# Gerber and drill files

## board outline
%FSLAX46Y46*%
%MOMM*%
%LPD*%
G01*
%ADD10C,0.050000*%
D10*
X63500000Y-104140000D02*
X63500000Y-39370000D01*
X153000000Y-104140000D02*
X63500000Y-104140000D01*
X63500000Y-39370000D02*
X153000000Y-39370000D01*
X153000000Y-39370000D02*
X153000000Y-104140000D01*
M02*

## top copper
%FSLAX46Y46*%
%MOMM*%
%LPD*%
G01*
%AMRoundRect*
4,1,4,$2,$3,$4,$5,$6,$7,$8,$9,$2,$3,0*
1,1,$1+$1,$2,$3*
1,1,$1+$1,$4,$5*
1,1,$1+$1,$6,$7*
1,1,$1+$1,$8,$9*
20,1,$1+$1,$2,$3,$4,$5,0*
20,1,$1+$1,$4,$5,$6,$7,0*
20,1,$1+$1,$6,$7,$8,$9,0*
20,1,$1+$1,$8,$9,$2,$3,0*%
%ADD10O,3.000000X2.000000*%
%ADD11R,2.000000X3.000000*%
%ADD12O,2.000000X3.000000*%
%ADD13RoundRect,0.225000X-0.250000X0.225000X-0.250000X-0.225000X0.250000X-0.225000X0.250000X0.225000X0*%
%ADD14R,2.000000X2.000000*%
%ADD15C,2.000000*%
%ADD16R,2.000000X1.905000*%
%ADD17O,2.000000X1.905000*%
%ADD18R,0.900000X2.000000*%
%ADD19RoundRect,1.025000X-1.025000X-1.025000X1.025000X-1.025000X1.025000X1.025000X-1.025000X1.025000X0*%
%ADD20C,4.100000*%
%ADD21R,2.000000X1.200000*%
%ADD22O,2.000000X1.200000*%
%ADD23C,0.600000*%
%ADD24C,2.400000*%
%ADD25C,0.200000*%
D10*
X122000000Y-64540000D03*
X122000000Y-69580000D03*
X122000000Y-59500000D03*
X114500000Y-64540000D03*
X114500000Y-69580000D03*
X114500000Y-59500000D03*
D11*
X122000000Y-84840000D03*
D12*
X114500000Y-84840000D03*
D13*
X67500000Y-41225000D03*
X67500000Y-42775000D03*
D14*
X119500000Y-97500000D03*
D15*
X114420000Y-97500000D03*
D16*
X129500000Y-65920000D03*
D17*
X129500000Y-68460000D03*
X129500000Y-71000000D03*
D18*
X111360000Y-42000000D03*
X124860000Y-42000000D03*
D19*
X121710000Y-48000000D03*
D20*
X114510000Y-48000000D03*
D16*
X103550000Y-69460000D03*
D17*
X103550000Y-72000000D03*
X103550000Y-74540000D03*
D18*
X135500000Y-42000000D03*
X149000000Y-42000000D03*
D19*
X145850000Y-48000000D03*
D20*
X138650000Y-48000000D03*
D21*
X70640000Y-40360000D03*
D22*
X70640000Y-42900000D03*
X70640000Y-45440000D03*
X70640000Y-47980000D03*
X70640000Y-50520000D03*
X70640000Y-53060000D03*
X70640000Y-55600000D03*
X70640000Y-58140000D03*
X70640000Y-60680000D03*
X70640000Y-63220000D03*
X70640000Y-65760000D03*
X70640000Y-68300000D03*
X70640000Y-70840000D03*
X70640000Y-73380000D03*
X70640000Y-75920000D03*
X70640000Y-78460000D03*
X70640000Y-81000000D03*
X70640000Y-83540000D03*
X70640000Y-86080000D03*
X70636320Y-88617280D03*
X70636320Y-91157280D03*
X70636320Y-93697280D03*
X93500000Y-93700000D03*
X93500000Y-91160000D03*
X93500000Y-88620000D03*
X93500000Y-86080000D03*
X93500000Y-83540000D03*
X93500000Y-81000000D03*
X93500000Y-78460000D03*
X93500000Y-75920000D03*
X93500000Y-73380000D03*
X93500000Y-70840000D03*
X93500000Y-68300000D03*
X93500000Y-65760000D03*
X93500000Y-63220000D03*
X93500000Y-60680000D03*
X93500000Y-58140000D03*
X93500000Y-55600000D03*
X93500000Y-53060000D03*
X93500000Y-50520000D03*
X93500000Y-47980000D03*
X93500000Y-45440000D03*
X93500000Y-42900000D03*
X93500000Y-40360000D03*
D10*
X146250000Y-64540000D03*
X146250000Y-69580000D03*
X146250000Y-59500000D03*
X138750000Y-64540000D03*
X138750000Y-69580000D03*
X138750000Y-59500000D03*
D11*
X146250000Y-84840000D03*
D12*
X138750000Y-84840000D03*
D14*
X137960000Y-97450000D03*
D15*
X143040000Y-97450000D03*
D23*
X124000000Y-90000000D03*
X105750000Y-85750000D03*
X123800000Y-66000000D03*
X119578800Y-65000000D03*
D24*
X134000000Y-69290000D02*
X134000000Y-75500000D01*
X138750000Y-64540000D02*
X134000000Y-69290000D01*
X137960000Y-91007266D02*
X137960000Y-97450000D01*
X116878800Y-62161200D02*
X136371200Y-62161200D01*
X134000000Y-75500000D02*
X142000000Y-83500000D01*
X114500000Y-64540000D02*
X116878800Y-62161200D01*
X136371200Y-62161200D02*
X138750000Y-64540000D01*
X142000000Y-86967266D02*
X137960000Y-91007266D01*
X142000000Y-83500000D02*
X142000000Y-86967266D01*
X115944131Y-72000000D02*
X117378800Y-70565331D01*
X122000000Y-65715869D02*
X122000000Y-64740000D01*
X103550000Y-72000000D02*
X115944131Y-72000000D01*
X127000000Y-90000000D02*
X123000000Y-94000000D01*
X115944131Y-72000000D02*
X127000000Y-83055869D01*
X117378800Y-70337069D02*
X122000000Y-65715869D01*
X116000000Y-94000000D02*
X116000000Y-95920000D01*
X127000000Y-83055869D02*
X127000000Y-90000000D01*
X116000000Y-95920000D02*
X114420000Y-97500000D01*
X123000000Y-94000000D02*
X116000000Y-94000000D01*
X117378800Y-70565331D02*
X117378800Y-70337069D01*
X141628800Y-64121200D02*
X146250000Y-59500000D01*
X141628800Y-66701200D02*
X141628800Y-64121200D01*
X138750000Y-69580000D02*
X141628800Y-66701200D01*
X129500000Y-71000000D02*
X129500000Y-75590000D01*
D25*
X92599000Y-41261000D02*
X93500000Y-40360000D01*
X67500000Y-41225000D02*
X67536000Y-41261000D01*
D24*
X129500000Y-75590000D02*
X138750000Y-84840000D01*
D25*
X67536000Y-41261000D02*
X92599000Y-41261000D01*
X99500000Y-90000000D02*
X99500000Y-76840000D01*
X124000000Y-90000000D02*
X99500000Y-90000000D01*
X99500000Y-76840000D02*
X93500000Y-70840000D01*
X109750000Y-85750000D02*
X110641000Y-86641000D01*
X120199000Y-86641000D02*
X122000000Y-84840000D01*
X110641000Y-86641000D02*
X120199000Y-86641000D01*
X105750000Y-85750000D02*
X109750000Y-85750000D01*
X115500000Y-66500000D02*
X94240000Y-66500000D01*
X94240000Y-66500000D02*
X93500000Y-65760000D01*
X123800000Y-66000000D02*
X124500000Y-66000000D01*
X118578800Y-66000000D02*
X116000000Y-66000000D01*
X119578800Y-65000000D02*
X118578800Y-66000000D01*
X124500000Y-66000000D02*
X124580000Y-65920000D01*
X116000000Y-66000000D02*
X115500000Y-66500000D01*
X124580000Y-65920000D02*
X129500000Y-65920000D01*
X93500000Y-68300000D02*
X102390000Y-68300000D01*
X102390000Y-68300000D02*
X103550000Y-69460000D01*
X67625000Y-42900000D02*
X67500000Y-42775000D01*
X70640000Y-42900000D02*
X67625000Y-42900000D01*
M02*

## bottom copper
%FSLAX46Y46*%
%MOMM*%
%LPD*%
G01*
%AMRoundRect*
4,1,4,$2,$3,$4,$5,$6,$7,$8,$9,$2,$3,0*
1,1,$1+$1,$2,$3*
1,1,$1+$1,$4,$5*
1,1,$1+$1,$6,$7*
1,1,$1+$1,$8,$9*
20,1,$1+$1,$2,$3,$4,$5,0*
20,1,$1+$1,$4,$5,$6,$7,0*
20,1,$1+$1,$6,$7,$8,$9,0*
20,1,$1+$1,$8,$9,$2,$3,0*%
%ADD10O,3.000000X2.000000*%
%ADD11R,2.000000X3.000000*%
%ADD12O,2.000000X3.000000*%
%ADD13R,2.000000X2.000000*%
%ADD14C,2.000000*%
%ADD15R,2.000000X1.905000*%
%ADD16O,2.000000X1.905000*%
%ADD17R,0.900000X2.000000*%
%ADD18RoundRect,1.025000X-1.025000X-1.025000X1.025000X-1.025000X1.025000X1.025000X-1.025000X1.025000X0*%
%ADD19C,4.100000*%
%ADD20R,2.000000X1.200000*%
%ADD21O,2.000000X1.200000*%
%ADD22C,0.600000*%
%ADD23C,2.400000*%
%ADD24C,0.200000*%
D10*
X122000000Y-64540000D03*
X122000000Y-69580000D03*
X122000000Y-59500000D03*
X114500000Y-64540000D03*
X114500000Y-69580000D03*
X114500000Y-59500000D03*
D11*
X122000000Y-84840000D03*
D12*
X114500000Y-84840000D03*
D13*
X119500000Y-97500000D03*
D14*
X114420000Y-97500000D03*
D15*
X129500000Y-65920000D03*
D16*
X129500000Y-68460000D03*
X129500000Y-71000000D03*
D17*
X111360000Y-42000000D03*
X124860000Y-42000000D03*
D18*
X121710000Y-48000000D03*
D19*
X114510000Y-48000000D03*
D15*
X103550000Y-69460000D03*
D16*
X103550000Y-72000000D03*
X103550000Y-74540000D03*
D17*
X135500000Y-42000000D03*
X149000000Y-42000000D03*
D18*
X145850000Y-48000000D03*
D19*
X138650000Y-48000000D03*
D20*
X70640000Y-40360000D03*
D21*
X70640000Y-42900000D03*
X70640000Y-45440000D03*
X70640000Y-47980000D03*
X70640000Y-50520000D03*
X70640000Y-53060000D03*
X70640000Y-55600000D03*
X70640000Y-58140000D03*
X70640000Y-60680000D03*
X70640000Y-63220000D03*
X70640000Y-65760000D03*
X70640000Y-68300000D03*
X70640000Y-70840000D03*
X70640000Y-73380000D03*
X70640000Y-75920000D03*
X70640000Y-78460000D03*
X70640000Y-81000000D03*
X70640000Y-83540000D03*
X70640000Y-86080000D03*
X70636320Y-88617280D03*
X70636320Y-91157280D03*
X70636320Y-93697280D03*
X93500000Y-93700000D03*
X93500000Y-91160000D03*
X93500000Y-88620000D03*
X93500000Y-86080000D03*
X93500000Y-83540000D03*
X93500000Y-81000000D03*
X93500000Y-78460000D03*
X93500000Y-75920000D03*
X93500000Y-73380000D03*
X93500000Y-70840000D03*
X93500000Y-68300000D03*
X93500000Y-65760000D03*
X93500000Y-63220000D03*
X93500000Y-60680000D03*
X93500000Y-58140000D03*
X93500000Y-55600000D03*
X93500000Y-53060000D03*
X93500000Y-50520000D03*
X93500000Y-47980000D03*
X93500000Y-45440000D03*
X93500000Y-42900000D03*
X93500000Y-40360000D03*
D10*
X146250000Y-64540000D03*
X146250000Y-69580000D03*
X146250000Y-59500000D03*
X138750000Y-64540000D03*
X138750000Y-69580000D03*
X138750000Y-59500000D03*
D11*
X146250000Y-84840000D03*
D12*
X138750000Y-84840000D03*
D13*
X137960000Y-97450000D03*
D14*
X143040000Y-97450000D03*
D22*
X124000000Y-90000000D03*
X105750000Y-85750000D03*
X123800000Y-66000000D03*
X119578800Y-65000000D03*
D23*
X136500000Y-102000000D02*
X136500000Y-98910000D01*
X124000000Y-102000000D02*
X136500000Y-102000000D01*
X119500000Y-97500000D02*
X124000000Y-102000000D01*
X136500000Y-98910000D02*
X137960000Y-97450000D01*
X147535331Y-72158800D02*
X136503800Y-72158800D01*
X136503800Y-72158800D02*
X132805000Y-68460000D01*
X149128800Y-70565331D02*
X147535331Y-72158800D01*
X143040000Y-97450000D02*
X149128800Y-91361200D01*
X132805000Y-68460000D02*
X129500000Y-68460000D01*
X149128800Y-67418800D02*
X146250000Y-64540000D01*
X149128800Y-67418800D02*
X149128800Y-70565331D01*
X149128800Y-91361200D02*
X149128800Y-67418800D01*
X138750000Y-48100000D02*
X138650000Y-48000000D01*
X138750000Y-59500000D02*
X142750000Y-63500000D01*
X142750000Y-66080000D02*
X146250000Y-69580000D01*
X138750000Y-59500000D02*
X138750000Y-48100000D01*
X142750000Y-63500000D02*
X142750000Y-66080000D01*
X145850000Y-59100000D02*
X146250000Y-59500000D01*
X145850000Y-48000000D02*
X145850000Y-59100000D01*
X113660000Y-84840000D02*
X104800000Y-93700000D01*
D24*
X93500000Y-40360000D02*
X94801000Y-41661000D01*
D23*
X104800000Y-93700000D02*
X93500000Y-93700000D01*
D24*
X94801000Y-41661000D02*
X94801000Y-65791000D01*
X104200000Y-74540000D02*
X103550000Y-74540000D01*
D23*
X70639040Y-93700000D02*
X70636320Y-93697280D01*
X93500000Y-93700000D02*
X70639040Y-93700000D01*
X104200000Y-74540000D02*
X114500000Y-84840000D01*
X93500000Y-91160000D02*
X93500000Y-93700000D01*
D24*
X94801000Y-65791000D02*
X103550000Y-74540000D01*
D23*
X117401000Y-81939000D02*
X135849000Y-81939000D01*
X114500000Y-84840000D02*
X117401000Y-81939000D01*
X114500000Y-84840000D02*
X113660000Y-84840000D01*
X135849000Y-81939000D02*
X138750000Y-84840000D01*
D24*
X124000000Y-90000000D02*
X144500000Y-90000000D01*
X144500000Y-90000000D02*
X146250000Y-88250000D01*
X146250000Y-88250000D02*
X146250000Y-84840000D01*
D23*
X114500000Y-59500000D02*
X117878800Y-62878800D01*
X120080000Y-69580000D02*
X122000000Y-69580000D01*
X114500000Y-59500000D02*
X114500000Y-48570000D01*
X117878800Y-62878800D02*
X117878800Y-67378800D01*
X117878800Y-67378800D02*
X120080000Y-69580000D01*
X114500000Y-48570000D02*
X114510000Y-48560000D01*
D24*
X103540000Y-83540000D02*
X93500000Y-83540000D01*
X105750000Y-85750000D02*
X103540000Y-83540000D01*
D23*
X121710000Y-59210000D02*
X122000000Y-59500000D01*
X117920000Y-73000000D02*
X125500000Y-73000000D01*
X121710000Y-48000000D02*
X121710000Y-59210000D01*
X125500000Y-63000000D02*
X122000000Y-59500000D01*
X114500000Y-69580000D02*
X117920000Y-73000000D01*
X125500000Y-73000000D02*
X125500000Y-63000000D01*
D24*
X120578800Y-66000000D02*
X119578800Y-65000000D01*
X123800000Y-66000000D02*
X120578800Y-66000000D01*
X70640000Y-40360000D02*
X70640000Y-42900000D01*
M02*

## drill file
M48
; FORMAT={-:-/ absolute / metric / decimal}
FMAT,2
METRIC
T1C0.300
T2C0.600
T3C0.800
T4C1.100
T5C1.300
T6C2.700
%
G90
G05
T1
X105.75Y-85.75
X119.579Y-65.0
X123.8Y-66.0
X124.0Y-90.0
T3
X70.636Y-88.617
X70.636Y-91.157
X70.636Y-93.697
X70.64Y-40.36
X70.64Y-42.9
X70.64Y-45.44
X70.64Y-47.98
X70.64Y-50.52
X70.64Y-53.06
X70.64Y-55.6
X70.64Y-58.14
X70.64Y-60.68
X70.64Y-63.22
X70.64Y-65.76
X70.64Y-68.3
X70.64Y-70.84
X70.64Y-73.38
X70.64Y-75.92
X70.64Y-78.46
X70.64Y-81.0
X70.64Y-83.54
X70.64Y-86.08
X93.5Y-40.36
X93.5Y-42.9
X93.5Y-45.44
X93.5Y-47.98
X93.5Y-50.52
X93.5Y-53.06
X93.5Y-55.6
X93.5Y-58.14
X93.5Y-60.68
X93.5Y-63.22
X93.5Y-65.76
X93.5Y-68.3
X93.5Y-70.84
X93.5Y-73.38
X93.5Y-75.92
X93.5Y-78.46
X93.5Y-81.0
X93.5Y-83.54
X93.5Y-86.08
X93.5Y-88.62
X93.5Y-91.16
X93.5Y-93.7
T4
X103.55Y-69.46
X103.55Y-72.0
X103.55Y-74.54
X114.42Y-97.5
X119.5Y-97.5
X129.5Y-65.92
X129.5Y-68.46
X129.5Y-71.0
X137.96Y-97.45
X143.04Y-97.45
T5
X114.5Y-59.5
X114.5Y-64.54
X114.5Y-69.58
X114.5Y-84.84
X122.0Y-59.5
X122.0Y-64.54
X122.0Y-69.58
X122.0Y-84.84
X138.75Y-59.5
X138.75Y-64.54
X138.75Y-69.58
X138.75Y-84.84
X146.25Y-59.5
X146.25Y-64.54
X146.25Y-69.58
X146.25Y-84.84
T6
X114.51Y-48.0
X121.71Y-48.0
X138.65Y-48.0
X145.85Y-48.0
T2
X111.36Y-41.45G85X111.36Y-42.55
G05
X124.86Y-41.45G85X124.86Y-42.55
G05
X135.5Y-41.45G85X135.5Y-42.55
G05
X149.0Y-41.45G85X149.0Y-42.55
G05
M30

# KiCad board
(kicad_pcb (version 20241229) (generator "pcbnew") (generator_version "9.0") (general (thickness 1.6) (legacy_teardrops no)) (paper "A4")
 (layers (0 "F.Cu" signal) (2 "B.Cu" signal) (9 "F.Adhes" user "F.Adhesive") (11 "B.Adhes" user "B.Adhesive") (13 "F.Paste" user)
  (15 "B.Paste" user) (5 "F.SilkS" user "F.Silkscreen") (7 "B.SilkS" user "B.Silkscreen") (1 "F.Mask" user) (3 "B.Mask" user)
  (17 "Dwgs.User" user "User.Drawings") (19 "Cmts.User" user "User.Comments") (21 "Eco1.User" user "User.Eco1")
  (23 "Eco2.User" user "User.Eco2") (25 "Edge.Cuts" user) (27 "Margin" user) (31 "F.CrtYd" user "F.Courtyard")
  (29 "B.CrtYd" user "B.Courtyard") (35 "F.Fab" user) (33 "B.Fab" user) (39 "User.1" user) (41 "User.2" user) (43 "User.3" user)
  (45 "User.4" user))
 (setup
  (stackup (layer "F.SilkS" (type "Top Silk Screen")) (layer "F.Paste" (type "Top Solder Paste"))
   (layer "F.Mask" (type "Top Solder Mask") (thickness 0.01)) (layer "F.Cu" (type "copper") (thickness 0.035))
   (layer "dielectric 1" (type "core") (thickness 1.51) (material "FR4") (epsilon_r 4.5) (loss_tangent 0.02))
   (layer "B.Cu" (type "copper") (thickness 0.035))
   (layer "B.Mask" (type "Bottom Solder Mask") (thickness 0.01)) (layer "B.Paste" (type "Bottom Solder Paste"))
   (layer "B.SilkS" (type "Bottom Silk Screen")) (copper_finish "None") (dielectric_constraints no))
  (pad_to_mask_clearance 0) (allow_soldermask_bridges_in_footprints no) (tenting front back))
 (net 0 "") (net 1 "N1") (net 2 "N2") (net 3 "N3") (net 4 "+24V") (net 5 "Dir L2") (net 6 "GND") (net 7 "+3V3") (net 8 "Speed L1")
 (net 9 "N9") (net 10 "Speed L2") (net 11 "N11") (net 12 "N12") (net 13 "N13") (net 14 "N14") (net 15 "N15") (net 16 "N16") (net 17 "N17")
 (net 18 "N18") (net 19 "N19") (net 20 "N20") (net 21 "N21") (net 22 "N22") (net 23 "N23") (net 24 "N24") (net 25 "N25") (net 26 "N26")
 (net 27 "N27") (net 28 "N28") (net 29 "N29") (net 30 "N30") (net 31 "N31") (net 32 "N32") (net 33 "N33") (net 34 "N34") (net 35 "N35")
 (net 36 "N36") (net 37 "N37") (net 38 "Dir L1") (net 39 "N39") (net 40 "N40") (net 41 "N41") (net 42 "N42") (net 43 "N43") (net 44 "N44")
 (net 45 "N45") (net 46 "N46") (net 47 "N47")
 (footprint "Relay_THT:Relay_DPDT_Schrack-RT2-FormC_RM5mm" (layer "F.Cu") (at 122 84.84 90)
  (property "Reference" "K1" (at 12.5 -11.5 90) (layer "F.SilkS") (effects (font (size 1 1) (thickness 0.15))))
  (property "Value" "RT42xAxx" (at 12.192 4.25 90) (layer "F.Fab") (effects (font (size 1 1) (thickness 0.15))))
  (pad "11" thru_hole oval (at 20.3 0 270) (size 2 3) (drill 1.3) (layers "*.Cu" "*.Mask") (remove_unused_layers no) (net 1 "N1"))
  (pad "12" thru_hole oval (at 15.26 0 270) (size 2 3) (drill 1.3) (layers "*.Cu" "*.Mask") (remove_unused_layers no) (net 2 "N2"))
  (pad "14" thru_hole oval (at 25.34 0 270) (size 2 3) (drill 1.3) (layers "*.Cu" "*.Mask") (remove_unused_layers no) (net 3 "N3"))
  (pad "21" thru_hole oval (at 20.3 -7.5 270) (size 2 3) (drill 1.3) (layers "*.Cu" "*.Mask") (remove_unused_layers no) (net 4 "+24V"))
  (pad "22" thru_hole oval (at 15.26 -7.5 270) (size 2 3) (drill 1.3) (layers "*.Cu" "*.Mask") (remove_unused_layers no) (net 3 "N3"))
  (pad "24" thru_hole oval (at 25.34 -7.5 270) (size 2 3) (drill 1.3) (layers "*.Cu" "*.Mask") (remove_unused_layers no) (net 2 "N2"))
  (pad "A1" thru_hole rect (at 0 0 270) (size 3 2) (drill 1.3) (layers "*.Cu" "*.Mask") (remove_unused_layers no) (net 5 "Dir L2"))
  (pad "A2" thru_hole oval (at 0 -7.5 270) (size 3 2) (drill 1.3) (layers "*.Cu" "*.Mask") (remove_unused_layers no) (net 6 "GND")))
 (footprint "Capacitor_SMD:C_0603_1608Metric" (layer "F.Cu") (at 67.5 42 -90)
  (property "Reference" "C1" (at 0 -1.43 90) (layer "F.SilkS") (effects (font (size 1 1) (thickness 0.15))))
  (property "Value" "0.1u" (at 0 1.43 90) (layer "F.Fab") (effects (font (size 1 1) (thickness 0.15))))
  (pad "1" smd roundrect (at -0.775 0 270) (size 0.9 0.95) (layers "F.Cu" "F.Mask" "F.Paste") (roundrect_rratio 0.25) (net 6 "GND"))
  (pad "2" smd roundrect (at 0.775 0 270) (size 0.9 0.95) (layers "F.Cu" "F.Mask" "F.Paste") (roundrect_rratio 0.25) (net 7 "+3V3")))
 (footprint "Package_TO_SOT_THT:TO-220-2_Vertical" (layer "F.Cu") (at 119.5 97.5 180)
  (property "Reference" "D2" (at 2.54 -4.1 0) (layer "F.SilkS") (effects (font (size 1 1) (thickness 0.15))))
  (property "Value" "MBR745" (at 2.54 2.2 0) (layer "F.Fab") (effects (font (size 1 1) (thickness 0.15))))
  (pad "1" thru_hole rect (at 0 0 180) (size 2 2) (drill 1.1) (layers "*.Cu" "*.Mask") (remove_unused_layers no) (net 4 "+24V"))
  (pad "2" thru_hole circle (at 5.08 0 180) (size 2 2) (drill 1.1) (layers "*.Cu" "*.Mask") (remove_unused_layers no) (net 1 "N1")))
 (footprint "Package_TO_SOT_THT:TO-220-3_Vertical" (layer "F.Cu") (at 129.5 65.92 -90)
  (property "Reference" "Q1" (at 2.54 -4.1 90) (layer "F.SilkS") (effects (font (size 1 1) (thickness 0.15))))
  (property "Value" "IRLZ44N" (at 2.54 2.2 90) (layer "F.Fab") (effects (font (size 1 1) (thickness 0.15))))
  (pad "1" thru_hole rect (at 0 0 270) (size 1.905 2) (drill 1.1) (layers "*.Cu" "*.Mask") (remove_unused_layers no) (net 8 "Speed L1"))
  (pad "2" thru_hole oval (at 2.54 0 270) (size 1.905 2) (drill 1.1) (layers "*.Cu" "*.Mask") (remove_unused_layers no) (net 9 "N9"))
  (pad "3" thru_hole oval (at 5.08 0 270) (size 1.905 2) (drill 1.1) (layers "*.Cu" "*.Mask") (remove_unused_layers no) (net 6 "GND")))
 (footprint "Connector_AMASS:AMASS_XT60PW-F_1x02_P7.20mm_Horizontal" (layer "F.Cu") (at 121.71 48)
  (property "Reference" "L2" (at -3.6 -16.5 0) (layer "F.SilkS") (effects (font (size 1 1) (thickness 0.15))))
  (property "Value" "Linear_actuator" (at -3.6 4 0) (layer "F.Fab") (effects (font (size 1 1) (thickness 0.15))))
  (pad "" thru_hole rect (at -10.35 -6) (size 0.9 2) (drill oval 0.6 1.7) (layers "*.Cu" "*.Mask") (remove_unused_layers no))
  (pad "" thru_hole rect (at 3.15 -6) (size 0.9 2) (drill oval 0.6 1.7) (layers "*.Cu" "*.Mask") (remove_unused_layers no))
  (pad "1" thru_hole roundrect (at 0 0) (size 4.1 4.1) (drill 2.7) (layers "*.Cu" "*.Mask") (remove_unused_layers no)
   (roundrect_rratio 0.25) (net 3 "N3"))
  (pad "2" thru_hole circle (at -7.2 0) (size 4.1 4.1) (drill 2.7) (layers "*.Cu" "*.Mask") (remove_unused_layers no) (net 2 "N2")))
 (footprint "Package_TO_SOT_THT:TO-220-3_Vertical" (layer "F.Cu") (at 103.55 69.46 -90)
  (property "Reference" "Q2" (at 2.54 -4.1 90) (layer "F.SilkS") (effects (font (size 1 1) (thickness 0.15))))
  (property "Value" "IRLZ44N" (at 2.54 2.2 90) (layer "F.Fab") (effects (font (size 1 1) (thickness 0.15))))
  (pad "1" thru_hole rect (at 0 0 270) (size 1.905 2) (drill 1.1) (layers "*.Cu" "*.Mask") (remove_unused_layers no) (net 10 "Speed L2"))
  (pad "2" thru_hole oval (at 2.54 0 270) (size 1.905 2) (drill 1.1) (layers "*.Cu" "*.Mask") (remove_unused_layers no) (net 1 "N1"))
  (pad "3" thru_hole oval (at 5.08 0 270) (size 1.905 2) (drill 1.1) (layers "*.Cu" "*.Mask") (remove_unused_layers no) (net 6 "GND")))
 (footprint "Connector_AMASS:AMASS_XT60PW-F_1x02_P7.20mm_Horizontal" (layer "F.Cu") (at 145.85 48)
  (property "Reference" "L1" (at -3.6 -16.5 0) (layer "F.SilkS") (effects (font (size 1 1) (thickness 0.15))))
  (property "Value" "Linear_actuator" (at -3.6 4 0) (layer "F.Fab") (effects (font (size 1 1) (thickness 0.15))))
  (pad "" thru_hole rect (at -10.35 -6) (size 0.9 2) (drill oval 0.6 1.7) (layers "*.Cu" "*.Mask") (remove_unused_layers no))
  (pad "" thru_hole rect (at 3.15 -6) (size 0.9 2) (drill oval 0.6 1.7) (layers "*.Cu" "*.Mask") (remove_unused_layers no))
  (pad "1" thru_hole roundrect (at 0 0) (size 4.1 4.1) (drill 2.7) (layers "*.Cu" "*.Mask") (remove_unused_layers no)
   (roundrect_rratio 0.25) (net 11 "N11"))
  (pad "2" thru_hole circle (at -7.2 0) (size 4.1 4.1) (drill 2.7) (layers "*.Cu" "*.Mask") (remove_unused_layers no) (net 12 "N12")))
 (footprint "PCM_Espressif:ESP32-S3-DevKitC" (layer "F.Cu") (at 70.64 40.36)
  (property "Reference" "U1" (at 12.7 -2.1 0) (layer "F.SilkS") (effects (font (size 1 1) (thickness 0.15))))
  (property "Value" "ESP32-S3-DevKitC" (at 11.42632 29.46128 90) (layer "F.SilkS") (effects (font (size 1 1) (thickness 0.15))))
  (pad "1" thru_hole rect (at 0 0 270) (size 1.2 2) (drill 0.8) (layers "*.Cu" "*.Mask") (remove_unused_layers no) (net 7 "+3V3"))
  (pad "2" thru_hole oval (at 0 2.54 270) (size 1.2 2) (drill 0.8) (layers "*.Cu" "*.Mask") (remove_unused_layers no) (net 7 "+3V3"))
  (pad "3" thru_hole oval (at 0 5.08 270) (size 1.2 2) (drill 0.8) (layers "*.Cu" "*.Mask") (remove_unused_layers no) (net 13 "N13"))
  (pad "4" thru_hole oval (at 0 7.62 270) (size 1.2 2) (drill 0.8) (layers "*.Cu" "*.Mask") (remove_unused_layers no) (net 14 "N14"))
  (pad "5" thru_hole oval (at 0 10.16 270) (size 1.2 2) (drill 0.8) (layers "*.Cu" "*.Mask") (remove_unused_layers no) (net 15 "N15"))
  (pad "6" thru_hole oval (at 0 12.7 270) (size 1.2 2) (drill 0.8) (layers "*.Cu" "*.Mask") (remove_unused_layers no) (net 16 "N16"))
  (pad "7" thru_hole oval (at 0 15.24 270) (size 1.2 2) (drill 0.8) (layers "*.Cu" "*.Mask") (remove_unused_layers no) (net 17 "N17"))
  (pad "8" thru_hole oval (at 0 17.78 270) (size 1.2 2) (drill 0.8) (layers "*.Cu" "*.Mask") (remove_unused_layers no) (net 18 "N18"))
  (pad "9" thru_hole oval (at 0 20.32 270) (size 1.2 2) (drill 0.8) (layers "*.Cu" "*.Mask") (remove_unused_layers no) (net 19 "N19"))
  (pad "10" thru_hole oval (at 0 22.86 270) (size 1.2 2) (drill 0.8) (layers "*.Cu" "*.Mask") (remove_unused_layers no) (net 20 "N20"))
  (pad "11" thru_hole oval (at 0 25.4 270) (size 1.2 2) (drill 0.8) (layers "*.Cu" "*.Mask") (remove_unused_layers no) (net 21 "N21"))
  (pad "12" thru_hole oval (at 0 27.94 270) (size 1.2 2) (drill 0.8) (layers "*.Cu" "*.Mask") (remove_unused_layers no) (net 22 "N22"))
  (pad "13" thru_hole oval (at 0 30.48 270) (size 1.2 2) (drill 0.8) (layers "*.Cu" "*.Mask") (remove_unused_layers no) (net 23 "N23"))
  (pad "14" thru_hole oval (at 0 33.02 270) (size 1.2 2) (drill 0.8) (layers "*.Cu" "*.Mask") (remove_unused_layers no) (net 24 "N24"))
  (pad "15" thru_hole oval (at 0 35.56 270) (size 1.2 2) (drill 0.8) (layers "*.Cu" "*.Mask") (remove_unused_layers no) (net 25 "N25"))
  (pad "16" thru_hole oval (at 0 38.1 270) (size 1.2 2) (drill 0.8) (layers "*.Cu" "*.Mask") (remove_unused_layers no) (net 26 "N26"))
  (pad "17" thru_hole oval (at 0 40.64 270) (size 1.2 2) (drill 0.8) (layers "*.Cu" "*.Mask") (remove_unused_layers no) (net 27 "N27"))
  (pad "18" thru_hole oval (at 0 43.18 270) (size 1.2 2) (drill 0.8) (layers "*.Cu" "*.Mask") (remove_unused_layers no) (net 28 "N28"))
  (pad "19" thru_hole oval (at 0 45.72 270) (size 1.2 2) (drill 0.8) (layers "*.Cu" "*.Mask") (remove_unused_layers no) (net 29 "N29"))
  (pad "20" thru_hole oval (at -0.00368 48.25728 270) (size 1.2 2) (drill 0.8) (layers "*.Cu" "*.Mask") (remove_unused_layers no)
   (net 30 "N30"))
  (pad "21" thru_hole oval (at -0.00368 50.79728 270) (size 1.2 2) (drill 0.8) (layers "*.Cu" "*.Mask") (remove_unused_layers no)
   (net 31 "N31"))
  (pad "22" thru_hole oval (at -0.00368 53.33728 270) (size 1.2 2) (drill 0.8) (layers "*.Cu" "*.Mask") (remove_unused_layers no)
   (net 6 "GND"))
  (pad "23" thru_hole oval (at 22.86 53.34 270) (size 1.2 2) (drill 0.8) (layers "*.Cu" "*.Mask") (remove_unused_layers no) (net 6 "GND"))
  (pad "24" thru_hole oval (at 22.86 50.8 270) (size 1.2 2) (drill 0.8) (layers "*.Cu" "*.Mask") (remove_unused_layers no) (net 6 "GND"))
  (pad "25" thru_hole oval (at 22.86 48.26 270) (size 1.2 2) (drill 0.8) (layers "*.Cu" "*.Mask") (remove_unused_layers no) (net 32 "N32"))
  (pad "26" thru_hole oval (at 22.86 45.72 270) (size 1.2 2) (drill 0.8) (layers "*.Cu" "*.Mask") (remove_unused_layers no) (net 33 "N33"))
  (pad "27" thru_hole oval (at 22.86 43.18 270) (size 1.2 2) (drill 0.8) (layers "*.Cu" "*.Mask") (remove_unused_layers no) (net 5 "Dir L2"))
  (pad "28" thru_hole oval (at 22.86 40.64 270) (size 1.2 2) (drill 0.8) (layers "*.Cu" "*.Mask") (remove_unused_layers no) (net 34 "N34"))
  (pad "29" thru_hole oval (at 22.86 38.1 270) (size 1.2 2) (drill 0.8) (layers "*.Cu" "*.Mask") (remove_unused_layers no) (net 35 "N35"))
  (pad "30" thru_hole oval (at 22.86 35.56 270) (size 1.2 2) (drill 0.8) (layers "*.Cu" "*.Mask") (remove_unused_layers no) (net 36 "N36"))
  (pad "31" thru_hole oval (at 22.86 33.02 270) (size 1.2 2) (drill 0.8) (layers "*.Cu" "*.Mask") (remove_unused_layers no) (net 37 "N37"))
  (pad "32" thru_hole oval (at 22.86 30.48 270) (size 1.2 2) (drill 0.8) (layers "*.Cu" "*.Mask") (remove_unused_layers no)
   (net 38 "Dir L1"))
  (pad "33" thru_hole oval (at 22.86 27.94 270) (size 1.2 2) (drill 0.8) (layers "*.Cu" "*.Mask") (remove_unused_layers no)
   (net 10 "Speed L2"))
  (pad "34" thru_hole oval (at 22.86 25.4 270) (size 1.2 2) (drill 0.8) (layers "*.Cu" "*.Mask") (remove_unused_layers no)
   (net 8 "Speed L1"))
  (pad "35" thru_hole oval (at 22.86 22.86 270) (size 1.2 2) (drill 0.8) (layers "*.Cu" "*.Mask") (remove_unused_layers no) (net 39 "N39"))
  (pad "36" thru_hole oval (at 22.86 20.32 270) (size 1.2 2) (drill 0.8) (layers "*.Cu" "*.Mask") (remove_unused_layers no) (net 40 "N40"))
  (pad "37" thru_hole oval (at 22.86 17.78 270) (size 1.2 2) (drill 0.8) (layers "*.Cu" "*.Mask") (remove_unused_layers no) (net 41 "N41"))
  (pad "38" thru_hole oval (at 22.86 15.24 270) (size 1.2 2) (drill 0.8) (layers "*.Cu" "*.Mask") (remove_unused_layers no) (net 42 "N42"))
  (pad "39" thru_hole oval (at 22.86 12.7 270) (size 1.2 2) (drill 0.8) (layers "*.Cu" "*.Mask") (remove_unused_layers no) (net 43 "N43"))
  (pad "40" thru_hole oval (at 22.86 10.16 270) (size 1.2 2) (drill 0.8) (layers "*.Cu" "*.Mask") (remove_unused_layers no) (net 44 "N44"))
  (pad "41" thru_hole oval (at 22.86 7.62 270) (size 1.2 2) (drill 0.8) (layers "*.Cu" "*.Mask") (remove_unused_layers no) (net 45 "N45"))
  (pad "42" thru_hole oval (at 22.86 5.08 270) (size 1.2 2) (drill 0.8) (layers "*.Cu" "*.Mask") (remove_unused_layers no) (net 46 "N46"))
  (pad "43" thru_hole oval (at 22.86 2.54 270) (size 1.2 2) (drill 0.8) (layers "*.Cu" "*.Mask") (remove_unused_layers no) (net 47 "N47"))
  (pad "44" thru_hole oval (at 22.86 0 270) (size 1.2 2) (drill 0.8) (layers "*.Cu" "*.Mask") (remove_unused_layers no) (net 6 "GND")))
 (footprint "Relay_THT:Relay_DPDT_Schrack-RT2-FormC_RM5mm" (layer "F.Cu") (at 146.25 84.84 90)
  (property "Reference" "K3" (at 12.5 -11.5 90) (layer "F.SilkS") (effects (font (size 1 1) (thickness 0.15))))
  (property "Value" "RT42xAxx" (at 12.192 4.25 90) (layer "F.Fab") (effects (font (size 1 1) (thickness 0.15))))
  (pad "11" thru_hole oval (at 20.3 0 270) (size 2 3) (drill 1.3) (layers "*.Cu" "*.Mask") (remove_unused_layers no) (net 9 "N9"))
  (pad "12" thru_hole oval (at 15.26 0 270) (size 2 3) (drill 1.3) (layers "*.Cu" "*.Mask") (remove_unused_layers no) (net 12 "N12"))
  (pad "14" thru_hole oval (at 25.34 0 270) (size 2 3) (drill 1.3) (layers "*.Cu" "*.Mask") (remove_unused_layers no) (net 11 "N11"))
  (pad "21" thru_hole oval (at 20.3 -7.5 270) (size 2 3) (drill 1.3) (layers "*.Cu" "*.Mask") (remove_unused_layers no) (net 4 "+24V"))
  (pad "22" thru_hole oval (at 15.26 -7.5 270) (size 2 3) (drill 1.3) (layers "*.Cu" "*.Mask") (remove_unused_layers no) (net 11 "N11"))
  (pad "24" thru_hole oval (at 25.34 -7.5 270) (size 2 3) (drill 1.3) (layers "*.Cu" "*.Mask") (remove_unused_layers no) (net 12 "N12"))
  (pad "A1" thru_hole rect (at 0 0 270) (size 3 2) (drill 1.3) (layers "*.Cu" "*.Mask") (remove_unused_layers no) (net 38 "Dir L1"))
  (pad "A2" thru_hole oval (at 0 -7.5 270) (size 3 2) (drill 1.3) (layers "*.Cu" "*.Mask") (remove_unused_layers no) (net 6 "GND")))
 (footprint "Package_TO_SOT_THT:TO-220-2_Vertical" (layer "F.Cu") (at 137.96 97.45)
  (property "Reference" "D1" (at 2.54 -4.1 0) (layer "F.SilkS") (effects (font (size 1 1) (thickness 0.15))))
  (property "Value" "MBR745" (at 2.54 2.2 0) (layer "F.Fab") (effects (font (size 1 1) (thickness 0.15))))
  (pad "1" thru_hole rect (at 0 0) (size 2 2) (drill 1.1) (layers "*.Cu" "*.Mask") (remove_unused_layers no) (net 4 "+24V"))
  (pad "2" thru_hole circle (at 5.08 0) (size 2 2) (drill 1.1) (layers "*.Cu" "*.Mask") (remove_unused_layers no) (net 9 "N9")))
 (gr_line (start 63.5 104.14) (end 63.5 39.37) (stroke (width 0.05) (type default)) (layer "Edge.Cuts"))
 (gr_line (start 153 104.14) (end 63.5 104.14) (stroke (width 0.05) (type default)) (layer "Edge.Cuts"))
 (gr_line (start 63.5 39.37) (end 153 39.37) (stroke (width 0.05) (type default)) (layer "Edge.Cuts"))
 (gr_line (start 153 39.37) (end 153 104.14) (stroke (width 0.05) (type default)) (layer "Edge.Cuts"))
 (segment (start 134 69.29) (end 134 75.5) (width 2.4) (layer "F.Cu") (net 4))
 (segment (start 138.75 64.54) (end 134 69.29) (width 2.4) (layer "F.Cu") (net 4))
 (segment (start 137.96 91.007266) (end 137.96 97.45) (width 2.4) (layer "F.Cu") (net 4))
 (segment (start 116.8788 62.1612) (end 136.3712 62.1612) (width 2.4) (layer "F.Cu") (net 4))
 (segment (start 134 75.5) (end 142 83.5) (width 2.4) (layer "F.Cu") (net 4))
 (segment (start 114.5 64.54) (end 116.8788 62.1612) (width 2.4) (layer "F.Cu") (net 4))
 (segment (start 136.3712 62.1612) (end 138.75 64.54) (width 2.4) (layer "F.Cu") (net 4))
 (segment (start 142 86.967266) (end 137.96 91.007266) (width 2.4) (layer "F.Cu") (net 4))
 (segment (start 142 83.5) (end 142 86.967266) (width 2.4) (layer "F.Cu") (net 4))
 (segment (start 136.5 102) (end 136.5 98.91) (width 2.4) (layer "B.Cu") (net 4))
 (segment (start 124 102) (end 136.5 102) (width 2.4) (layer "B.Cu") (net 4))
 (segment (start 119.5 97.5) (end 124 102) (width 2.4) (layer "B.Cu") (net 4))
 (segment (start 136.5 98.91) (end 137.96 97.45) (width 2.4) (layer "B.Cu") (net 4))
 (segment (start 147.535331 72.1588) (end 136.5038 72.1588) (width 2.4) (layer "B.Cu") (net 9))
 (segment (start 136.5038 72.1588) (end 132.805 68.46) (width 2.4) (layer "B.Cu") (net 9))
 (segment (start 149.1288 70.565331) (end 147.535331 72.1588) (width 2.4) (layer "B.Cu") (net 9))
 (segment (start 143.04 97.45) (end 149.1288 91.3612) (width 2.4) (layer "B.Cu") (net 9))
 (segment (start 132.805 68.46) (end 129.5 68.46) (width 2.4) (layer "B.Cu") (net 9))
 (segment (start 149.1288 67.4188) (end 146.25 64.54) (width 2.4) (layer "B.Cu") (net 9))
 (segment (start 149.1288 67.4188) (end 149.1288 70.565331) (width 2.4) (layer "B.Cu") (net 9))
 (segment (start 149.1288 91.3612) (end 149.1288 67.4188) (width 2.4) (layer "B.Cu") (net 9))
 (segment (start 115.944131 72) (end 117.3788 70.565331) (width 2.4) (layer "F.Cu") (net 1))
 (segment (start 122 65.715869) (end 122 64.74) (width 2.4) (layer "F.Cu") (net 1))
 (segment (start 103.55 72) (end 115.944131 72) (width 2.4) (layer "F.Cu") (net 1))
 (segment (start 127 90) (end 123 94) (width 2.4) (layer "F.Cu") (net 1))
 (segment (start 115.944131 72) (end 127 83.055869) (width 2.4) (layer "F.Cu") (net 1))
 (segment (start 117.3788 70.337069) (end 122 65.715869) (width 2.4) (layer "F.Cu") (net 1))
 (segment (start 116 94) (end 116 95.92) (width 2.4) (layer "F.Cu") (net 1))
 (segment (start 127 83.055869) (end 127 90) (width 2.4) (layer "F.Cu") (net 1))
 (segment (start 116 95.92) (end 114.42 97.5) (width 2.4) (layer "F.Cu") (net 1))
 (segment (start 123 94) (end 116 94) (width 2.4) (layer "F.Cu") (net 1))
 (segment (start 117.3788 70.565331) (end 117.3788 70.337069) (width 2.4) (layer "F.Cu") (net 1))
 (segment (start 138.75 48.1) (end 138.65 48) (width 2.4) (layer "B.Cu") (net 12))
 (segment (start 138.75 59.5) (end 142.75 63.5) (width 2.4) (layer "B.Cu") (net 12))
 (segment (start 142.75 66.08) (end 146.25 69.58) (width 2.4) (layer "B.Cu") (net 12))
 (segment (start 138.75 59.5) (end 138.75 48.1) (width 2.4) (layer "B.Cu") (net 12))
 (segment (start 142.75 63.5) (end 142.75 66.08) (width 2.4) (layer "B.Cu") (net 12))
 (segment (start 141.6288 64.1212) (end 146.25 59.5) (width 2.4) (layer "F.Cu") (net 11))
 (segment (start 141.6288 66.7012) (end 141.6288 64.1212) (width 2.4) (layer "F.Cu") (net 11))
 (segment (start 138.75 69.58) (end 141.6288 66.7012) (width 2.4) (layer "F.Cu") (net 11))
 (segment (start 145.85 59.1) (end 146.25 59.5) (width 2.4) (layer "B.Cu") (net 11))
 (segment (start 145.85 48) (end 145.85 59.1) (width 2.4) (layer "B.Cu") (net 11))
 (segment (start 129.5 71) (end 129.5 75.59) (width 2.4) (layer "F.Cu") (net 6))
 (segment (start 92.599 41.261) (end 93.5 40.36) (width 0.2) (layer "F.Cu") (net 6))
 (segment (start 67.5 41.225) (end 67.536 41.261) (width 0.2) (layer "F.Cu") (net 6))
 (segment (start 129.5 75.59) (end 138.75 84.84) (width 2.4) (layer "F.Cu") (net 6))
 (segment (start 67.536 41.261) (end 92.599 41.261) (width 0.2) (layer "F.Cu") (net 6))
 (segment (start 113.66 84.84) (end 104.8 93.7) (width 2.4) (layer "B.Cu") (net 6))
 (segment (start 93.5 40.36) (end 94.801 41.661) (width 0.2) (layer "B.Cu") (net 6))
 (segment (start 104.8 93.7) (end 93.5 93.7) (width 2.4) (layer "B.Cu") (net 6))
 (segment (start 94.801 41.661) (end 94.801 65.791) (width 0.2) (layer "B.Cu") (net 6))
 (segment (start 104.2 74.54) (end 103.55 74.54) (width 0.2) (layer "B.Cu") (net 6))
 (segment (start 70.63904 93.7) (end 70.63632 93.69728) (width 2.4) (layer "B.Cu") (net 6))
 (segment (start 93.5 93.7) (end 70.63904 93.7) (width 2.4) (layer "B.Cu") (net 6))
 (segment (start 104.2 74.54) (end 114.5 84.84) (width 2.4) (layer "B.Cu") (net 6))
 (segment (start 93.5 91.16) (end 93.5 93.7) (width 2.4) (layer "B.Cu") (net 6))
 (segment (start 94.801 65.791) (end 103.55 74.54) (width 0.2) (layer "B.Cu") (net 6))
 (segment (start 117.401 81.939) (end 135.849 81.939) (width 2.4) (layer "B.Cu") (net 6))
 (segment (start 114.5 84.84) (end 117.401 81.939) (width 2.4) (layer "B.Cu") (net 6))
 (segment (start 114.5 84.84) (end 113.66 84.84) (width 2.4) (layer "B.Cu") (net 6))
 (segment (start 135.849 81.939) (end 138.75 84.84) (width 2.4) (layer "B.Cu") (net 6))
 (segment (start 99.5 90) (end 99.5 76.84) (width 0.2) (layer "F.Cu") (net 38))
 (segment (start 124 90) (end 99.5 90) (width 0.2) (layer "F.Cu") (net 38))
 (segment (start 99.5 76.84) (end 93.5 70.84) (width 0.2) (layer "F.Cu") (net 38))
 (via (at 124 90) (size 0.6) (drill 0.3) (layers "F.Cu" "B.Cu") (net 38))
 (segment (start 124 90) (end 144.5 90) (width 0.2) (layer "B.Cu") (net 38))
 (segment (start 144.5 90) (end 146.25 88.25) (width 0.2) (layer "B.Cu") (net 38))
 (segment (start 146.25 88.25) (end 146.25 84.84) (width 0.2) (layer "B.Cu") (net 38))
 (segment (start 114.5 59.5) (end 117.8788 62.8788) (width 2.4) (layer "B.Cu") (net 2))
 (segment (start 120.08 69.58) (end 122 69.58) (width 2.4) (layer "B.Cu") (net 2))
 (segment (start 114.5 59.5) (end 114.5 48.57) (width 2.4) (layer "B.Cu") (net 2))
 (segment (start 117.8788 62.8788) (end 117.8788 67.3788) (width 2.4) (layer "B.Cu") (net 2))
 (segment (start 117.8788 67.3788) (end 120.08 69.58) (width 2.4) (layer "B.Cu") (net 2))
 (segment (start 114.5 48.57) (end 114.51 48.56) (width 2.4) (layer "B.Cu") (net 2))
 (segment (start 109.75 85.75) (end 110.641 86.641) (width 0.2) (layer "F.Cu") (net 5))
 (segment (start 120.199 86.641) (end 122 84.84) (width 0.2) (layer "F.Cu") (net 5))
 (segment (start 110.641 86.641) (end 120.199 86.641) (width 0.2) (layer "F.Cu") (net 5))
 (segment (start 105.75 85.75) (end 109.75 85.75) (width 0.2) (layer "F.Cu") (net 5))
 (via (at 105.75 85.75) (size 0.6) (drill 0.3) (layers "F.Cu" "B.Cu") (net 5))
 (segment (start 103.54 83.54) (end 93.5 83.54) (width 0.2) (layer "B.Cu") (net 5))
 (segment (start 105.75 85.75) (end 103.54 83.54) (width 0.2) (layer "B.Cu") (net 5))
 (segment (start 121.71 59.21) (end 122 59.5) (width 2.4) (layer "B.Cu") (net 3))
 (segment (start 117.92 73) (end 125.5 73) (width 2.4) (layer "B.Cu") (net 3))
 (segment (start 121.71 48) (end 121.71 59.21) (width 2.4) (layer "B.Cu") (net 3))
 (segment (start 125.5 63) (end 122 59.5) (width 2.4) (layer "B.Cu") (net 3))
 (segment (start 114.5 69.58) (end 117.92 73) (width 2.4) (layer "B.Cu") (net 3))
 (segment (start 125.5 73) (end 125.5 63) (width 2.4) (layer "B.Cu") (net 3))
 (segment (start 115.5 66.5) (end 94.24 66.5) (width 0.2) (layer "F.Cu") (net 8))
 (segment (start 94.24 66.5) (end 93.5 65.76) (width 0.2) (layer "F.Cu") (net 8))
 (segment (start 123.8 66) (end 124.5 66) (width 0.2) (layer "F.Cu") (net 8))
 (segment (start 118.5788 66) (end 116 66) (width 0.2) (layer "F.Cu") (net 8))
 (segment (start 119.5788 65) (end 118.5788 66) (width 0.2) (layer "F.Cu") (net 8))
 (segment (start 124.5 66) (end 124.58 65.92) (width 0.2) (layer "F.Cu") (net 8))
 (segment (start 116 66) (end 115.5 66.5) (width 0.2) (layer "F.Cu") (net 8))
 (segment (start 124.58 65.92) (end 129.5 65.92) (width 0.2) (layer "F.Cu") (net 8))
 (via (at 123.8 66) (size 0.6) (drill 0.3) (layers "F.Cu" "B.Cu") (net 8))
 (via (at 119.5788 65) (size 0.6) (drill 0.3) (layers "F.Cu" "B.Cu") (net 8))
 (segment (start 120.5788 66) (end 119.5788 65) (width 0.2) (layer "B.Cu") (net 8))
 (segment (start 123.8 66) (end 120.5788 66) (width 0.2) (layer "B.Cu") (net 8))
 (segment (start 93.5 68.3) (end 102.39 68.3) (width 0.2) (layer "F.Cu") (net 10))
 (segment (start 102.39 68.3) (end 103.55 69.46) (width 0.2) (layer "F.Cu") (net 10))
 (segment (start 67.625 42.9) (end 67.5 42.775) (width 0.2) (layer "F.Cu") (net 7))
 (segment (start 70.64 42.9) (end 67.625 42.9) (width 0.2) (layer "F.Cu") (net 7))
 (segment (start 70.64 40.36) (end 70.64 42.9) (width 0.2) (layer "B.Cu") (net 7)))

